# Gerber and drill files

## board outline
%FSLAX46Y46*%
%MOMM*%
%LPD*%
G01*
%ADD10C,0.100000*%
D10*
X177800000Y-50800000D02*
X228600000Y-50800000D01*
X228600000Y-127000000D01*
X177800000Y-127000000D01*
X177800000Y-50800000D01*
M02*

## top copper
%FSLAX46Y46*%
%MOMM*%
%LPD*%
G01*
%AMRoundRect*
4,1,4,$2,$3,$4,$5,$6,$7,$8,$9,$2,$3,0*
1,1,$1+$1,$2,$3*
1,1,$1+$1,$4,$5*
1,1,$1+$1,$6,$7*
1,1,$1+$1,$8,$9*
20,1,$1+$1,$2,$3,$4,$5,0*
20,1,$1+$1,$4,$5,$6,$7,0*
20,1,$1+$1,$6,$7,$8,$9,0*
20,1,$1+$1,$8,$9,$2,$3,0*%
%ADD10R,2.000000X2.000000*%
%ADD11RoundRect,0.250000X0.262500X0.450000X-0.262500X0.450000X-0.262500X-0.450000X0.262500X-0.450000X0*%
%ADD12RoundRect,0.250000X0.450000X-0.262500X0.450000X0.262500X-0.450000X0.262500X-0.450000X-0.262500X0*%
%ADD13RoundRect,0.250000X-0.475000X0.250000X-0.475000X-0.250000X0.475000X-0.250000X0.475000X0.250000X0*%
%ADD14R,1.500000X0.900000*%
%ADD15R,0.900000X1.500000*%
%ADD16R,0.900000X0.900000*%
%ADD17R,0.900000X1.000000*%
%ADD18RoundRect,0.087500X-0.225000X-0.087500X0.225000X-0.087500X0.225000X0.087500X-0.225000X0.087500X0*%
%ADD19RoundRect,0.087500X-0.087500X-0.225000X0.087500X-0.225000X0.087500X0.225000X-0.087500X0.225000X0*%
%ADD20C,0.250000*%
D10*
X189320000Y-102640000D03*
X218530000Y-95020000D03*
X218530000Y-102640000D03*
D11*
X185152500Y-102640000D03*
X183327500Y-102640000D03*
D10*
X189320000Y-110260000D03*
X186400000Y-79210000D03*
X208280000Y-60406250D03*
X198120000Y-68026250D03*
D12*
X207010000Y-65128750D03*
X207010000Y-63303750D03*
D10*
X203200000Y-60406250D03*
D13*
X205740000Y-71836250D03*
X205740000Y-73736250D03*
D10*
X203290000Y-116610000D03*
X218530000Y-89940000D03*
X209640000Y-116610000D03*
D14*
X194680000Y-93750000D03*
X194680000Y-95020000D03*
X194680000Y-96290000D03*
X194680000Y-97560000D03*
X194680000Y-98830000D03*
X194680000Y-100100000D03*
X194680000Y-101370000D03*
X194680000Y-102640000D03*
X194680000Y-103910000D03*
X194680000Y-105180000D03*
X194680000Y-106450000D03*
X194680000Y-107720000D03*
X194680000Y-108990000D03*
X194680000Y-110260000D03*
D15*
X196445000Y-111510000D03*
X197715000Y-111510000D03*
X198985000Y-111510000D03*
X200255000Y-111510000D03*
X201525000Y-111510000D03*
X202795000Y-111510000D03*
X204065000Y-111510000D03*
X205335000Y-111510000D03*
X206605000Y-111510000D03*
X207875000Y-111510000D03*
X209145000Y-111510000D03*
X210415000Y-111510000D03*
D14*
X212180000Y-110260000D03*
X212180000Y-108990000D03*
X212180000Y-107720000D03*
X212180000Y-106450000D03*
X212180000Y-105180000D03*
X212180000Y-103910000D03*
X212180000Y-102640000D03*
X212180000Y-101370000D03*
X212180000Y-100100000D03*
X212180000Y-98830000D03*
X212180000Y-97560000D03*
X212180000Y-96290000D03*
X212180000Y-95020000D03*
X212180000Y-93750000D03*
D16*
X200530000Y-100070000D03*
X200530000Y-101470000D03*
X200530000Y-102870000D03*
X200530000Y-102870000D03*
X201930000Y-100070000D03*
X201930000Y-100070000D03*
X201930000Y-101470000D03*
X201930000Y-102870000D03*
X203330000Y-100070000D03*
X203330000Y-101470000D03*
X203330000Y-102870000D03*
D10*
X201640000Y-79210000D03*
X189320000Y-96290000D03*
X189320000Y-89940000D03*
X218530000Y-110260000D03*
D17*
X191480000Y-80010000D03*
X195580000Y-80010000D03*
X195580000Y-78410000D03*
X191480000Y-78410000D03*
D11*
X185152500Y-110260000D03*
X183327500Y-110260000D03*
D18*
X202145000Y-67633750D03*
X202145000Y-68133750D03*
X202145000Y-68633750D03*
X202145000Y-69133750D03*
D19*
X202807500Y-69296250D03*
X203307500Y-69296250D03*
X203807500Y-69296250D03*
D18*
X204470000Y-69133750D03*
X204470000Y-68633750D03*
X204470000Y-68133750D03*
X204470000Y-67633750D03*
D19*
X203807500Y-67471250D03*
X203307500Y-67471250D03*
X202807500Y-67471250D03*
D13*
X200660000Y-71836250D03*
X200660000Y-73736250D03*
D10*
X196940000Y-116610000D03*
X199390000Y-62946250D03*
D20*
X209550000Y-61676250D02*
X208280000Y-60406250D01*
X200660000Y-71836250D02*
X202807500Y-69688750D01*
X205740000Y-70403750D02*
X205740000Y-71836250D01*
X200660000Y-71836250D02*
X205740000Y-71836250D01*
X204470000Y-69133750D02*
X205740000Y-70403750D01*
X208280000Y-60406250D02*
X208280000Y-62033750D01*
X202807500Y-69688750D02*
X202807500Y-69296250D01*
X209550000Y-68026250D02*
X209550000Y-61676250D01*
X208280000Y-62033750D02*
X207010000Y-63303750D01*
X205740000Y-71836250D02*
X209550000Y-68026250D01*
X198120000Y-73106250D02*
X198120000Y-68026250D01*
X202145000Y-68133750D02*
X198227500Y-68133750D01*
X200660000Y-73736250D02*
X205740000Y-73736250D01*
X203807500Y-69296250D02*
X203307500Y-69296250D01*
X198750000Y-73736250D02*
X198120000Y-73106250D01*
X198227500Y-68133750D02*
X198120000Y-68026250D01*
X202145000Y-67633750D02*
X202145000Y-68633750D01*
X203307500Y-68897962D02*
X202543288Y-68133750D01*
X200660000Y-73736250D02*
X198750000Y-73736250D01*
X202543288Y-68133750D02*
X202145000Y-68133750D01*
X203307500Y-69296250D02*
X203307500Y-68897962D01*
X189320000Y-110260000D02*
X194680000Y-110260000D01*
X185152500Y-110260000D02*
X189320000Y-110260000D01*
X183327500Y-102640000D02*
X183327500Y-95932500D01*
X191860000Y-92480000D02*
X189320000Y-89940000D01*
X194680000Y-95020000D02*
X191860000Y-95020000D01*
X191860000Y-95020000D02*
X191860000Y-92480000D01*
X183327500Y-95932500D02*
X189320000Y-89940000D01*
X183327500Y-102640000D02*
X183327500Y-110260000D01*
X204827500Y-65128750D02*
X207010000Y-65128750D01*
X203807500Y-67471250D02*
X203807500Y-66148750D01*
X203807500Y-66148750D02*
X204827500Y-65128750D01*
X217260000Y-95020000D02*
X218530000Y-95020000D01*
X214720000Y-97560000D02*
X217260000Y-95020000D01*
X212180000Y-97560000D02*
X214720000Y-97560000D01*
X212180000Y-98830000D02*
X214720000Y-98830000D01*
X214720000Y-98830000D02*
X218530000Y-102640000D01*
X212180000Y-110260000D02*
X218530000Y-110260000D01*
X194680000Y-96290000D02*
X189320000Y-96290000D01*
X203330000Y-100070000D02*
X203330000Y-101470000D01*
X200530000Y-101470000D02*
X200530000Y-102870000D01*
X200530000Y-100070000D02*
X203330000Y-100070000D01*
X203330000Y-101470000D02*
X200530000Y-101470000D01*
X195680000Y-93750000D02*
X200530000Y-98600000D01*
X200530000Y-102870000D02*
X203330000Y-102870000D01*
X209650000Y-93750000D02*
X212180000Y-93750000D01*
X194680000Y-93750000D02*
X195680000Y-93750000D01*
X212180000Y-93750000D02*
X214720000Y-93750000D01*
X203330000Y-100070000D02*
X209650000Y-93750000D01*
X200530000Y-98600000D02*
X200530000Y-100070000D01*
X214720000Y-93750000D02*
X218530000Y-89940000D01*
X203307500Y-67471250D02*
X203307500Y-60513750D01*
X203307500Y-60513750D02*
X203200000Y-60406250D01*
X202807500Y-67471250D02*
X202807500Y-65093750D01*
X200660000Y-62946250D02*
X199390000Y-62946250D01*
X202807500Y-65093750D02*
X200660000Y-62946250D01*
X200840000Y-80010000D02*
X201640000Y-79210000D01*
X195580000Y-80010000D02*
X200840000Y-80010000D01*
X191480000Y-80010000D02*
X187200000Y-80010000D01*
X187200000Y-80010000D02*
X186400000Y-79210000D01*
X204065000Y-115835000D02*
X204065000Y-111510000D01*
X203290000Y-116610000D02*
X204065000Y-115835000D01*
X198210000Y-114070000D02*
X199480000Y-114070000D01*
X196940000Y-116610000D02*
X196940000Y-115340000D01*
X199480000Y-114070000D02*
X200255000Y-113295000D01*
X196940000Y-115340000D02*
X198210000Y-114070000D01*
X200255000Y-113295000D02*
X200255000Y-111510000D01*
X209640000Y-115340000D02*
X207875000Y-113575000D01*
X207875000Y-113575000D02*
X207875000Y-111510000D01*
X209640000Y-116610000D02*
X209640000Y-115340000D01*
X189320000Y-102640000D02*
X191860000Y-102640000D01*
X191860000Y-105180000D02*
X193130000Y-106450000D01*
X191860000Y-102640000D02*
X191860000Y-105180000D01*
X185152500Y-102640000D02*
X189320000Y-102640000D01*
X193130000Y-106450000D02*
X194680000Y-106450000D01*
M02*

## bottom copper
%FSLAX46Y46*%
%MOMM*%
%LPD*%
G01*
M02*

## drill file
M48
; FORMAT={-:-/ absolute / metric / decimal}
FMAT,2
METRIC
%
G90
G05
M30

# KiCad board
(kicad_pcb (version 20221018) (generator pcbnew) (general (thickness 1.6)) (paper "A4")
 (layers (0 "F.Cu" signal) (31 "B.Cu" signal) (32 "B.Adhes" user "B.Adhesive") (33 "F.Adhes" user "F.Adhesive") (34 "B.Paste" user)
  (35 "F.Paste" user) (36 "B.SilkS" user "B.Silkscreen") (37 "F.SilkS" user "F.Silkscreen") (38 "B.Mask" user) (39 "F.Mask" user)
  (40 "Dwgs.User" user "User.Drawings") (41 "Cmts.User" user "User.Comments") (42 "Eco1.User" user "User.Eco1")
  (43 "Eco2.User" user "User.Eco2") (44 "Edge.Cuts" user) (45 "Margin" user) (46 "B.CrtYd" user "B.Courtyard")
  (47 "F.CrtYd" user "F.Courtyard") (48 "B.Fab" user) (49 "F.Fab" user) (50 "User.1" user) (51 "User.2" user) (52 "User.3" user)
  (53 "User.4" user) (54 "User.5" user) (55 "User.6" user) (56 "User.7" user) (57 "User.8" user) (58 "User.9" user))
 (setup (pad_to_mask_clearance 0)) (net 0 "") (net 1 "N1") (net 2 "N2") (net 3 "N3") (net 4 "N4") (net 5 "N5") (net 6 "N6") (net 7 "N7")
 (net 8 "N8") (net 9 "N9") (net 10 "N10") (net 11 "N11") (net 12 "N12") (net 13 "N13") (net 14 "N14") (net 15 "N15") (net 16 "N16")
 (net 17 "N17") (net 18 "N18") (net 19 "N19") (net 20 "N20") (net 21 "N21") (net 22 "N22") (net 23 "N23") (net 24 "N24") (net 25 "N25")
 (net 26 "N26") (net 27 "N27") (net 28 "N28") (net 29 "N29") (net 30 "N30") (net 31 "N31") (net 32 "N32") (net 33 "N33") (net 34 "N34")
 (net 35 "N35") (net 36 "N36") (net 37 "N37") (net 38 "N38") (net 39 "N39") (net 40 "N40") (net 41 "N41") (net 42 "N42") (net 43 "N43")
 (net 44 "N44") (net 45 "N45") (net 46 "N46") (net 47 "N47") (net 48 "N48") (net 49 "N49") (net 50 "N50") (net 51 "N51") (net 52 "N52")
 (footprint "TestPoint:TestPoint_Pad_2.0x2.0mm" (layer "F.Cu") (at 189.32 102.64)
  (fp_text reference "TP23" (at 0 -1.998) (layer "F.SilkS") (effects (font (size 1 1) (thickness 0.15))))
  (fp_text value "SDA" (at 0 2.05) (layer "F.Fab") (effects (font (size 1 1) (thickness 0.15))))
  (pad "1" smd rect (at 0 0) (size 2 2) (layers "F.Cu" "F.Mask") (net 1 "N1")))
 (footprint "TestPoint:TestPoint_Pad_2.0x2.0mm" (layer "F.Cu") (at 218.53 95.02)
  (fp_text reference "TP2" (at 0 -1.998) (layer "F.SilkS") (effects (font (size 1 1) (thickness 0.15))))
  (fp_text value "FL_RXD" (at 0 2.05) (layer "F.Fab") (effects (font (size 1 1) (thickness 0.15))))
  (pad "1" smd rect (at 0 0) (size 2 2) (layers "F.Cu" "F.Mask") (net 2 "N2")))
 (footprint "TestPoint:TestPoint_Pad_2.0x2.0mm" (layer "F.Cu") (at 218.53 102.64)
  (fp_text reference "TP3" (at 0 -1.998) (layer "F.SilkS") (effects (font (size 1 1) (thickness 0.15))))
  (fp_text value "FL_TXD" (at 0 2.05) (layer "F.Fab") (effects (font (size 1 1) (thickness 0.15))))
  (pad "1" smd rect (at 0 0) (size 2 2) (layers "F.Cu" "F.Mask") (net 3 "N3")))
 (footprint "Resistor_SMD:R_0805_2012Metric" (layer "F.Cu") (at 184.24 102.64 180)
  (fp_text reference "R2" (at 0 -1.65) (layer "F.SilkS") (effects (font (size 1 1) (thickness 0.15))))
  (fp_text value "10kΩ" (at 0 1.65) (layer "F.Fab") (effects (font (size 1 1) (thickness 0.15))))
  (pad "1" smd roundrect (at -0.9125 0 180) (size 1.025 1.4) (layers "F.Cu" "F.Paste" "F.Mask") (roundrect_rratio 0.243902) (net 1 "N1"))
  (pad "2" smd roundrect (at 0.9125 0 180) (size 1.025 1.4) (layers "F.Cu" "F.Paste" "F.Mask") (roundrect_rratio 0.243902) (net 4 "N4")))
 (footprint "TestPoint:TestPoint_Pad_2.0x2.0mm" (layer "F.Cu") (at 189.32 110.26)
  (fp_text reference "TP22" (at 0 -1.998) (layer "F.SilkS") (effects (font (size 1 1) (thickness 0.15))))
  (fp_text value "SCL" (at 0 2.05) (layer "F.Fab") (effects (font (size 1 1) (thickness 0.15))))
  (pad "1" smd rect (at 0 0) (size 2 2) (layers "F.Cu" "F.Mask") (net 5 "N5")))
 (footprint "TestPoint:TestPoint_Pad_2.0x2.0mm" (layer "F.Cu") (at 186.4 79.21)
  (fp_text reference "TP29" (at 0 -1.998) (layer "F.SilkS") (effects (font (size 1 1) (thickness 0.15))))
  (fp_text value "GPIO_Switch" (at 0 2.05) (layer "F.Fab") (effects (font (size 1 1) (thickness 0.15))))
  (pad "1" smd rect (at 0 0) (size 2 2) (layers "F.Cu" "F.Mask") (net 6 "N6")))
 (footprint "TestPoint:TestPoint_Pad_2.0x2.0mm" (layer "F.Cu") (at 208.28 60.40625)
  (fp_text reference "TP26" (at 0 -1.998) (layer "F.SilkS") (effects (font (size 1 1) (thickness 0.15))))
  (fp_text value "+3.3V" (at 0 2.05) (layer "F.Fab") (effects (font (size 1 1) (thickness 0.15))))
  (pad "1" smd rect (at 0 0) (size 2 2) (layers "F.Cu" "F.Mask") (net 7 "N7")))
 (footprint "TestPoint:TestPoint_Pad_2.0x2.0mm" (layer "F.Cu") (at 198.12 68.02625)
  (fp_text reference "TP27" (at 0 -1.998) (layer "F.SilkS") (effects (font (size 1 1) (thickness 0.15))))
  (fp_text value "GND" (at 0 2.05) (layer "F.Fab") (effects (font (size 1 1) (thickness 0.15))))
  (pad "1" smd rect (at 0 0) (size 2 2) (layers "F.Cu" "F.Mask") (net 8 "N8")))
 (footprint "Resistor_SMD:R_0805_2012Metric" (layer "F.Cu") (at 207.01 64.21625 90)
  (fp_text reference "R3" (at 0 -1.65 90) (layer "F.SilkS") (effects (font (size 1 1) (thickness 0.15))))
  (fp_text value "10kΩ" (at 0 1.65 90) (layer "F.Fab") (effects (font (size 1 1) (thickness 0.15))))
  (pad "1" smd roundrect (at -0.9125 0 90) (size 1.025 1.4) (layers "F.Cu" "F.Paste" "F.Mask") (roundrect_rratio 0.243902) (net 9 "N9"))
  (pad "2" smd roundrect (at 0.9125 0 90) (size 1.025 1.4) (layers "F.Cu" "F.Paste" "F.Mask") (roundrect_rratio 0.243902) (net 7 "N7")))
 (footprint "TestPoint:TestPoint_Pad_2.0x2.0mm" (layer "F.Cu") (at 203.2 60.40625)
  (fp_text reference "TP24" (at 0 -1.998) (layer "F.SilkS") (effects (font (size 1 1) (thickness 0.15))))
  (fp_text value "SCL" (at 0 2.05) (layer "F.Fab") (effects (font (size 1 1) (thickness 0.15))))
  (pad "1" smd rect (at 0 0) (size 2 2) (layers "F.Cu" "F.Mask") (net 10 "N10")))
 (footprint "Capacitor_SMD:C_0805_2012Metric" (layer "F.Cu") (at 205.74 72.78625 -90)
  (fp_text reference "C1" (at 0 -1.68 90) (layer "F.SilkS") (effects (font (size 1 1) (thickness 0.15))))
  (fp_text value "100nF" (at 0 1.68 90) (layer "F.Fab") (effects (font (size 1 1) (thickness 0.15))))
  (pad "1" smd roundrect (at -0.95 0 270) (size 1 1.45) (layers "F.Cu" "F.Paste" "F.Mask") (roundrect_rratio 0.25) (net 7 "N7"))
  (pad "2" smd roundrect (at 0.95 0 270) (size 1 1.45) (layers "F.Cu" "F.Paste" "F.Mask") (roundrect_rratio 0.25) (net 8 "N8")))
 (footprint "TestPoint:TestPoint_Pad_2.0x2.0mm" (layer "F.Cu") (at 203.29 116.61)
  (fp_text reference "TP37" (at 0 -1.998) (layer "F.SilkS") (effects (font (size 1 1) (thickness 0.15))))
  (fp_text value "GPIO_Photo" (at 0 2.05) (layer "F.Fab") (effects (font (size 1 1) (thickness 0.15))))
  (pad "1" smd rect (at 0 0) (size 2 2) (layers "F.Cu" "F.Mask") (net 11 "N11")))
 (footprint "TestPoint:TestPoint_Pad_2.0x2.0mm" (layer "F.Cu") (at 218.53 89.94)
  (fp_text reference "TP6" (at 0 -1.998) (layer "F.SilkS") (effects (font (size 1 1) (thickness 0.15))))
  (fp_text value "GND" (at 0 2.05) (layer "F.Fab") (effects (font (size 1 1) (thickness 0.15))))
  (pad "1" smd rect (at 0 0) (size 2 2) (layers "F.Cu" "F.Mask") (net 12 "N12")))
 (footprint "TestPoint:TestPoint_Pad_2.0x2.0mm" (layer "F.Cu") (at 209.64 116.61)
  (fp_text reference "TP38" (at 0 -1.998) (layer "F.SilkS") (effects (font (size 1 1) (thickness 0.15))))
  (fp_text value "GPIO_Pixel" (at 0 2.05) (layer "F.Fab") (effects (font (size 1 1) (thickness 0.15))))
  (pad "1" smd rect (at 0 0) (size 2 2) (layers "F.Cu" "F.Mask") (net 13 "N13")))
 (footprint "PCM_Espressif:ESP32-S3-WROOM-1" (layer "F.Cu") (at 203.43 102.01)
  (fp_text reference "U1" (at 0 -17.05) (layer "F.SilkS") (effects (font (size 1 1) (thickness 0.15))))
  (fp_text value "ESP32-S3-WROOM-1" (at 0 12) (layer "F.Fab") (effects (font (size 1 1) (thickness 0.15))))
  (pad "1" smd rect (at -8.75 -8.26) (size 1.5 0.9) (layers "F.Cu" "F.Paste" "F.Mask") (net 12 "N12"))
  (pad "2" smd rect (at -8.75 -6.99) (size 1.5 0.9) (layers "F.Cu" "F.Paste" "F.Mask") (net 4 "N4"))
  (pad "3" smd rect (at -8.75 -5.72) (size 1.5 0.9) (layers "F.Cu" "F.Paste" "F.Mask") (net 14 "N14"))
  (pad "4" smd rect (at -8.75 -4.45) (size 1.5 0.9) (layers "F.Cu" "F.Paste" "F.Mask") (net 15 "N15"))
  (pad "5" smd rect (at -8.75 -3.18) (size 1.5 0.9) (layers "F.Cu" "F.Paste" "F.Mask") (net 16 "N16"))
  (pad "6" smd rect (at -8.75 -1.91) (size 1.5 0.9) (layers "F.Cu" "F.Paste" "F.Mask") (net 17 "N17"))
  (pad "7" smd rect (at -8.75 -0.64) (size 1.5 0.9) (layers "F.Cu" "F.Paste" "F.Mask") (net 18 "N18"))
  (pad "8" smd rect (at -8.75 0.63) (size 1.5 0.9) (layers "F.Cu" "F.Paste" "F.Mask") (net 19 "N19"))
  (pad "9" smd rect (at -8.75 1.9) (size 1.5 0.9) (layers "F.Cu" "F.Paste" "F.Mask") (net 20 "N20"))
  (pad "10" smd rect (at -8.75 3.17) (size 1.5 0.9) (layers "F.Cu" "F.Paste" "F.Mask") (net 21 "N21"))
  (pad "11" smd rect (at -8.75 4.44) (size 1.5 0.9) (layers "F.Cu" "F.Paste" "F.Mask") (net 1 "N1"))
  (pad "12" smd rect (at -8.75 5.71) (size 1.5 0.9) (layers "F.Cu" "F.Paste" "F.Mask") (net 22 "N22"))
  (pad "13" smd rect (at -8.75 6.98) (size 1.5 0.9) (layers "F.Cu" "F.Paste" "F.Mask") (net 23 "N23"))
  (pad "14" smd rect (at -8.75 8.25) (size 1.5 0.9) (layers "F.Cu" "F.Paste" "F.Mask") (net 5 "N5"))
  (pad "15" smd rect (at -6.985 9.5 90) (size 1.5 0.9) (layers "F.Cu" "F.Paste" "F.Mask") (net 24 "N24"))
  (pad "16" smd rect (at -5.715 9.5 90) (size 1.5 0.9) (layers "F.Cu" "F.Paste" "F.Mask") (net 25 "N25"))
  (pad "17" smd rect (at -4.445 9.5 90) (size 1.5 0.9) (layers "F.Cu" "F.Paste" "F.Mask") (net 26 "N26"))
  (pad "18" smd rect (at -3.175 9.5 90) (size 1.5 0.9) (layers "F.Cu" "F.Paste" "F.Mask") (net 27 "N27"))
  (pad "19" smd rect (at -1.905 9.5 90) (size 1.5 0.9) (layers "F.Cu" "F.Paste" "F.Mask") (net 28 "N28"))
  (pad "20" smd rect (at -0.635 9.5 90) (size 1.5 0.9) (layers "F.Cu" "F.Paste" "F.Mask") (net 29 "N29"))
  (pad "21" smd rect (at 0.635 9.5 90) (size 1.5 0.9) (layers "F.Cu" "F.Paste" "F.Mask") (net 11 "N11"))
  (pad "22" smd rect (at 1.905 9.5 90) (size 1.5 0.9) (layers "F.Cu" "F.Paste" "F.Mask") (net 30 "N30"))
  (pad "23" smd rect (at 3.175 9.5 90) (size 1.5 0.9) (layers "F.Cu" "F.Paste" "F.Mask") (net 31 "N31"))
  (pad "24" smd rect (at 4.445 9.5 90) (size 1.5 0.9) (layers "F.Cu" "F.Paste" "F.Mask") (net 13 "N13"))
  (pad "25" smd rect (at 5.715 9.5 90) (size 1.5 0.9) (layers "F.Cu" "F.Paste" "F.Mask") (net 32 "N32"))
  (pad "26" smd rect (at 6.985 9.5 90) (size 1.5 0.9) (layers "F.Cu" "F.Paste" "F.Mask") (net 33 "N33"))
  (pad "27" smd rect (at 8.75 8.25 180) (size 1.5 0.9) (layers "F.Cu" "F.Paste" "F.Mask") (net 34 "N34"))
  (pad "28" smd rect (at 8.75 6.98 180) (size 1.5 0.9) (layers "F.Cu" "F.Paste" "F.Mask") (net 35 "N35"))
  (pad "29" smd rect (at 8.75 5.71 180) (size 1.5 0.9) (layers "F.Cu" "F.Paste" "F.Mask") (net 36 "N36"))
  (pad "30" smd rect (at 8.75 4.44 180) (size 1.5 0.9) (layers "F.Cu" "F.Paste" "F.Mask") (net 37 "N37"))
  (pad "31" smd rect (at 8.75 3.17 180) (size 1.5 0.9) (layers "F.Cu" "F.Paste" "F.Mask") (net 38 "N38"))
  (pad "32" smd rect (at 8.75 1.9 180) (size 1.5 0.9) (layers "F.Cu" "F.Paste" "F.Mask") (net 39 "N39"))
  (pad "33" smd rect (at 8.75 0.63 180) (size 1.5 0.9) (layers "F.Cu" "F.Paste" "F.Mask") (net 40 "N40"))
  (pad "34" smd rect (at 8.75 -0.64 180) (size 1.5 0.9) (layers "F.Cu" "F.Paste" "F.Mask") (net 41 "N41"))
  (pad "35" smd rect (at 8.75 -1.91 180) (size 1.5 0.9) (layers "F.Cu" "F.Paste" "F.Mask") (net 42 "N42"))
  (pad "36" smd rect (at 8.75 -3.18 180) (size 1.5 0.9) (layers "F.Cu" "F.Paste" "F.Mask") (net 3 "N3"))
  (pad "37" smd rect (at 8.75 -4.45 180) (size 1.5 0.9) (layers "F.Cu" "F.Paste" "F.Mask") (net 2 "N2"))
  (pad "38" smd rect (at 8.75 -5.72 180) (size 1.5 0.9) (layers "F.Cu" "F.Paste" "F.Mask") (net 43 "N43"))
  (pad "39" smd rect (at 8.75 -6.99 180) (size 1.5 0.9) (layers "F.Cu" "F.Paste" "F.Mask") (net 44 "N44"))
  (pad "40" smd rect (at 8.75 -8.26 180) (size 1.5 0.9) (layers "F.Cu" "F.Paste" "F.Mask") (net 12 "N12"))
  (pad "41" smd rect (at -2.9 -1.94 180) (size 0.9 0.9) (layers "F.Cu" "F.Paste" "F.Mask") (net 12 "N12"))
  (pad "41" smd rect (at -2.9 -0.54 180) (size 0.9 0.9) (layers "F.Cu" "F.Paste" "F.Mask") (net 12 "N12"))
  (pad "41" smd rect (at -2.9 0.86 180) (size 0.9 0.9) (layers "F.Cu" "F.Paste" "F.Mask") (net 12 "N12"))
  (pad "41" smd rect (at -2.9 0.86 180) (size 0.9 0.9) (layers "F.Cu" "F.Paste" "F.Mask") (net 12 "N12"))
  (pad "41" smd rect (at -1.5 -1.94 180) (size 0.9 0.9) (layers "F.Cu" "F.Paste" "F.Mask") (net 12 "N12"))
  (pad "41" smd rect (at -1.5 -1.94 180) (size 0.9 0.9) (layers "F.Cu" "F.Paste" "F.Mask") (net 12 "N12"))
  (pad "41" smd rect (at -1.5 -0.54 180) (size 0.9 0.9) (layers "F.Cu" "F.Paste" "F.Mask") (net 12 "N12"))
  (pad "41" smd rect (at -1.5 0.86 180) (size 0.9 0.9) (layers "F.Cu" "F.Paste" "F.Mask") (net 12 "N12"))
  (pad "41" smd rect (at -0.1 -1.94 180) (size 0.9 0.9) (layers "F.Cu" "F.Paste" "F.Mask") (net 12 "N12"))
  (pad "41" smd rect (at -0.1 -0.54 180) (size 0.9 0.9) (layers "F.Cu" "F.Paste" "F.Mask") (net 12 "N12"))
  (pad "41" smd rect (at -0.1 0.86 180) (size 0.9 0.9) (layers "F.Cu" "F.Paste" "F.Mask") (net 12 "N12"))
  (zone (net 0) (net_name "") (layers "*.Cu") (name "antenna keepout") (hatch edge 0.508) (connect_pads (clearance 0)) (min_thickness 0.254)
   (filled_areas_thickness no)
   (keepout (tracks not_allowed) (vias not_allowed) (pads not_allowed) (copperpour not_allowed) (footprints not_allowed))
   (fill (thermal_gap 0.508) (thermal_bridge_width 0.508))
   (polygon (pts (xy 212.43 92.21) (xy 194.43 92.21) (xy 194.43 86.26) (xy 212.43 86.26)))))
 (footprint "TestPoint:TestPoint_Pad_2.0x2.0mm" (layer "F.Cu") (at 201.64 79.21)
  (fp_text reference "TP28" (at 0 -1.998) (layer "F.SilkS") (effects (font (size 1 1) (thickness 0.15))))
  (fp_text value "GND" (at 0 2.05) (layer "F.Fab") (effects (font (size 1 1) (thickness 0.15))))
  (pad "1" smd rect (at 0 0) (size 2 2) (layers "F.Cu" "F.Mask") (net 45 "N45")))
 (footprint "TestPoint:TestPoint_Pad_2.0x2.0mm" (layer "F.Cu") (at 189.32 96.29)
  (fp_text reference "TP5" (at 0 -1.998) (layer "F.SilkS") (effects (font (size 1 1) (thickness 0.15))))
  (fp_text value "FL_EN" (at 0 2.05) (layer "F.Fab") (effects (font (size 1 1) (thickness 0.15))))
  (pad "1" smd rect (at 0 0) (size 2 2) (layers "F.Cu" "F.Mask") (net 14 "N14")))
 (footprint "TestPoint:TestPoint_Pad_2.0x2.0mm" (layer "F.Cu") (at 189.32 89.94)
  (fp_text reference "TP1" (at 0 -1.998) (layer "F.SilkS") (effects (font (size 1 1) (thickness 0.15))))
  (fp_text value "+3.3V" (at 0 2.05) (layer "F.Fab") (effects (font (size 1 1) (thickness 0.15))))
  (pad "1" smd rect (at 0 0) (size 2 2) (layers "F.Cu" "F.Mask") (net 4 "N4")))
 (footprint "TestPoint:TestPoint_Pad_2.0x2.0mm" (layer "F.Cu") (at 218.53 110.26)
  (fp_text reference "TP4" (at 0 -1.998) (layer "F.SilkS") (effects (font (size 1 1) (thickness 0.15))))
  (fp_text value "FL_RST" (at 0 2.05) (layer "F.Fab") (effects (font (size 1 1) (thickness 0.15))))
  (pad "1" smd rect (at 0 0) (size 2 2) (layers "F.Cu" "F.Mask") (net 34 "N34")))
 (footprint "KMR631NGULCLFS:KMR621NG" (layer "F.Cu") (at 193.53 79.21)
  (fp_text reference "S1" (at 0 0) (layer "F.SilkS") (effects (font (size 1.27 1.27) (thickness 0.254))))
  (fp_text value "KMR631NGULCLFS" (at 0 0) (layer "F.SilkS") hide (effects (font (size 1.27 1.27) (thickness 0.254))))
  (pad "1" smd rect (at -2.05 0.8) (size 0.9 1) (layers "F.Cu" "F.Paste" "F.Mask") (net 6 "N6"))
  (pad "2" smd rect (at 2.05 0.8) (size 0.9 1) (layers "F.Cu" "F.Paste" "F.Mask") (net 45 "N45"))
  (pad "3" smd rect (at 2.05 -0.8) (size 0.9 1) (layers "F.Cu" "F.Paste" "F.Mask") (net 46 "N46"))
  (pad "4" smd rect (at -2.05 -0.8) (size 0.9 1) (layers "F.Cu" "F.Paste" "F.Mask") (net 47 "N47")))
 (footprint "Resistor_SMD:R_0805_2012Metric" (layer "F.Cu") (at 184.24 110.26 180)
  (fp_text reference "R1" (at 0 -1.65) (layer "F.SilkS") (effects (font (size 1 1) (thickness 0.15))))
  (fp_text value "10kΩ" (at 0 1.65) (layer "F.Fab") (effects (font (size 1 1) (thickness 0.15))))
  (pad "1" smd roundrect (at -0.9125 0 180) (size 1.025 1.4) (layers "F.Cu" "F.Paste" "F.Mask") (roundrect_rratio 0.243902) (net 5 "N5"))
  (pad "2" smd roundrect (at 0.9125 0 180) (size 1.025 1.4) (layers "F.Cu" "F.Paste" "F.Mask") (roundrect_rratio 0.243902) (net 4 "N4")))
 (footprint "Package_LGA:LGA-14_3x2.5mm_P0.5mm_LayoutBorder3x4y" (layer "F.Cu") (at 203.3075 68.38375)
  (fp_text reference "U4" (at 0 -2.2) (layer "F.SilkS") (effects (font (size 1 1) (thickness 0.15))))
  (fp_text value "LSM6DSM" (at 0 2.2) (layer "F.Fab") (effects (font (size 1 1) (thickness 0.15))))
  (pad "1" smd roundrect (at -1.1625 -0.75) (size 0.625 0.35) (layers "F.Cu" "F.Paste" "F.Mask") (roundrect_rratio 0.25) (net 8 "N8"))
  (pad "2" smd roundrect (at -1.1625 -0.25) (size 0.625 0.35) (layers "F.Cu" "F.Paste" "F.Mask") (roundrect_rratio 0.25) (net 8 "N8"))
  (pad "3" smd roundrect (at -1.1625 0.25) (size 0.625 0.35) (layers "F.Cu" "F.Paste" "F.Mask") (roundrect_rratio 0.25) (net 8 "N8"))
  (pad "4" smd roundrect (at -1.1625 0.75) (size 0.625 0.35) (layers "F.Cu" "F.Paste" "F.Mask") (roundrect_rratio 0.25) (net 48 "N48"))
  (pad "5" smd roundrect (at -0.5 0.9125) (size 0.35 0.625) (layers "F.Cu" "F.Paste" "F.Mask") (roundrect_rratio 0.25) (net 7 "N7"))
  (pad "6" smd roundrect (at 0 0.9125) (size 0.35 0.625) (layers "F.Cu" "F.Paste" "F.Mask") (roundrect_rratio 0.25) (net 8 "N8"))
  (pad "7" smd roundrect (at 0.5 0.9125) (size 0.35 0.625) (layers "F.Cu" "F.Paste" "F.Mask") (roundrect_rratio 0.25) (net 8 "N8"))
  (pad "8" smd roundrect (at 1.1625 0.75) (size 0.625 0.35) (layers "F.Cu" "F.Paste" "F.Mask") (roundrect_rratio 0.25) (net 7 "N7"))
  (pad "9" smd roundrect (at 1.1625 0.25) (size 0.625 0.35) (layers "F.Cu" "F.Paste" "F.Mask") (roundrect_rratio 0.25) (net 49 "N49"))
  (pad "10" smd roundrect (at 1.1625 -0.25) (size 0.625 0.35) (layers "F.Cu" "F.Paste" "F.Mask") (roundrect_rratio 0.25) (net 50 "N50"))
  (pad "11" smd roundrect (at 1.1625 -0.75) (size 0.625 0.35) (layers "F.Cu" "F.Paste" "F.Mask") (roundrect_rratio 0.25) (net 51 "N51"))
  (pad "12" smd roundrect (at 0.5 -0.9125) (size 0.35 0.625) (layers "F.Cu" "F.Paste" "F.Mask") (roundrect_rratio 0.25) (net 9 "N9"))
  (pad "13" smd roundrect (at 0 -0.9125) (size 0.35 0.625) (layers "F.Cu" "F.Paste" "F.Mask") (roundrect_rratio 0.25) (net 10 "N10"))
  (pad "14" smd roundrect (at -0.5 -0.9125) (size 0.35 0.625) (layers "F.Cu" "F.Paste" "F.Mask") (roundrect_rratio 0.25) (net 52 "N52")))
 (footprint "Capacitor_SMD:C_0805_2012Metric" (layer "F.Cu") (at 200.66 72.78625 -90)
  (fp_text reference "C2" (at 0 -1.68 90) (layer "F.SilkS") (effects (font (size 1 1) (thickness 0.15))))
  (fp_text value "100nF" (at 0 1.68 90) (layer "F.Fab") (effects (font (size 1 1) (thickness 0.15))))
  (pad "1" smd roundrect (at -0.95 0 270) (size 1 1.45) (layers "F.Cu" "F.Paste" "F.Mask") (roundrect_rratio 0.25) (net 7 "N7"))
  (pad "2" smd roundrect (at 0.95 0 270) (size 1 1.45) (layers "F.Cu" "F.Paste" "F.Mask") (roundrect_rratio 0.25) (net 8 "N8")))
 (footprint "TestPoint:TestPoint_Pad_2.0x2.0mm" (layer "F.Cu") (at 196.94 116.61)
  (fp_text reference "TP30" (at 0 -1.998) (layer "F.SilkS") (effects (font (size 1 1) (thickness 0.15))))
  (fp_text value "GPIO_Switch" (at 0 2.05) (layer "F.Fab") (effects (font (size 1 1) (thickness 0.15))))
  (pad "1" smd rect (at 0 0) (size 2 2) (layers "F.Cu" "F.Mask") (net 27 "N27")))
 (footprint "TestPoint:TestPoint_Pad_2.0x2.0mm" (layer "F.Cu") (at 199.39 62.94625)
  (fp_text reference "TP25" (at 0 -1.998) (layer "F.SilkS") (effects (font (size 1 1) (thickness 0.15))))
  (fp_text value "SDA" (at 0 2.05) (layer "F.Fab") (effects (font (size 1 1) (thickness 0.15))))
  (pad "1" smd rect (at 0 0) (size 2 2) (layers "F.Cu" "F.Mask") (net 52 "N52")))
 (gr_rect (start 177.8 50.8) (end 228.6 127) (stroke (width 0.1) (type default)) (fill none) (layer "Edge.Cuts"))
 (segment (start 209.55 61.67625) (end 208.28 60.40625) (width 0.25) (layer "F.Cu") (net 7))
 (segment (start 200.66 71.83625) (end 202.8075 69.68875) (width 0.25) (layer "F.Cu") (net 7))
 (segment (start 205.74 70.40375) (end 205.74 71.83625) (width 0.25) (layer "F.Cu") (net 7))
 (segment (start 200.66 71.83625) (end 205.74 71.83625) (width 0.25) (layer "F.Cu") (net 7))
 (segment (start 204.47 69.13375) (end 205.74 70.40375) (width 0.25) (layer "F.Cu") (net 7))
 (segment (start 208.28 60.40625) (end 208.28 62.03375) (width 0.25) (layer "F.Cu") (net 7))
 (segment (start 202.8075 69.68875) (end 202.8075 69.29625) (width 0.25) (layer "F.Cu") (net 7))
 (segment (start 209.55 68.02625) (end 209.55 61.67625) (width 0.25) (layer "F.Cu") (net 7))
 (segment (start 208.28 62.03375) (end 207.01 63.30375) (width 0.25) (layer "F.Cu") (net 7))
 (segment (start 205.74 71.83625) (end 209.55 68.02625) (width 0.25) (layer "F.Cu") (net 7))
 (segment (start 198.12 73.10625) (end 198.12 68.02625) (width 0.25) (layer "F.Cu") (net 8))
 (segment (start 202.145 68.13375) (end 198.2275 68.13375) (width 0.25) (layer "F.Cu") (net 8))
 (segment (start 200.66 73.73625) (end 205.74 73.73625) (width 0.25) (layer "F.Cu") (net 8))
 (segment (start 203.8075 69.29625) (end 203.3075 69.29625) (width 0.25) (layer "F.Cu") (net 8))
 (segment (start 198.75 73.73625) (end 198.12 73.10625) (width 0.25) (layer "F.Cu") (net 8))
 (segment (start 198.2275 68.13375) (end 198.12 68.02625) (width 0.25) (layer "F.Cu") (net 8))
 (segment (start 202.145 67.63375) (end 202.145 68.63375) (width 0.25) (layer "F.Cu") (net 8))
 (segment (start 203.3075 68.897962) (end 202.543288 68.13375) (width 0.25) (layer "F.Cu") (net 8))
 (segment (start 200.66 73.73625) (end 198.75 73.73625) (width 0.25) (layer "F.Cu") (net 8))
 (segment (start 202.543288 68.13375) (end 202.145 68.13375) (width 0.25) (layer "F.Cu") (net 8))
 (segment (start 203.3075 69.29625) (end 203.3075 68.897962) (width 0.25) (layer "F.Cu") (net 8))
 (segment (start 189.32 110.26) (end 194.68 110.26) (width 0.25) (layer "F.Cu") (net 5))
 (segment (start 185.1525 110.26) (end 189.32 110.26) (width 0.25) (layer "F.Cu") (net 5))
 (segment (start 183.3275 102.64) (end 183.3275 95.9325) (width 0.25) (layer "F.Cu") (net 4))
 (segment (start 191.86 92.48) (end 189.32 89.94) (width 0.25) (layer "F.Cu") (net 4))
 (segment (start 194.68 95.02) (end 191.86 95.02) (width 0.25) (layer "F.Cu") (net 4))
 (segment (start 191.86 95.02) (end 191.86 92.48) (width 0.25) (layer "F.Cu") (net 4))
 (segment (start 183.3275 95.9325) (end 189.32 89.94) (width 0.25) (layer "F.Cu") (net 4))
 (segment (start 183.3275 102.64) (end 183.3275 110.26) (width 0.25) (layer "F.Cu") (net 4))
 (segment (start 204.8275 65.12875) (end 207.01 65.12875) (width 0.25) (layer "F.Cu") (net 9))
 (segment (start 203.8075 67.47125) (end 203.8075 66.14875) (width 0.25) (layer "F.Cu") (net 9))
 (segment (start 203.8075 66.14875) (end 204.8275 65.12875) (width 0.25) (layer "F.Cu") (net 9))
 (segment (start 217.26 95.02) (end 218.53 95.02) (width 0.25) (layer "F.Cu") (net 2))
 (segment (start 214.72 97.56) (end 217.26 95.02) (width 0.25) (layer "F.Cu") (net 2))
 (segment (start 212.18 97.56) (end 214.72 97.56) (width 0.25) (layer "F.Cu") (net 2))
 (segment (start 212.18 98.83) (end 214.72 98.83) (width 0.25) (layer "F.Cu") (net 3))
 (segment (start 214.72 98.83) (end 218.53 102.64) (width 0.25) (layer "F.Cu") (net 3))
 (segment (start 212.18 110.26) (end 218.53 110.26) (width 0.25) (layer "F.Cu") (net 34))
 (segment (start 194.68 96.29) (end 189.32 96.29) (width 0.25) (layer "F.Cu") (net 14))
 (segment (start 203.33 100.07) (end 203.33 101.47) (width 0.25) (layer "F.Cu") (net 12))
 (segment (start 200.53 101.47) (end 200.53 102.87) (width 0.25) (layer "F.Cu") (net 12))
 (segment (start 200.53 100.07) (end 203.33 100.07) (width 0.25) (layer "F.Cu") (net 12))
 (segment (start 203.33 101.47) (end 200.53 101.47) (width 0.25) (layer "F.Cu") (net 12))
 (segment (start 195.68 93.75) (end 200.53 98.6) (width 0.25) (layer "F.Cu") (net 12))
 (segment (start 200.53 102.87) (end 203.33 102.87) (width 0.25) (layer "F.Cu") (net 12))
 (segment (start 209.65 93.75) (end 212.18 93.75) (width 0.25) (layer "F.Cu") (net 12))
 (segment (start 194.68 93.75) (end 195.68 93.75) (width 0.25) (layer "F.Cu") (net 12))
 (segment (start 212.18 93.75) (end 214.72 93.75) (width 0.25) (layer "F.Cu") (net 12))
 (segment (start 203.33 100.07) (end 209.65 93.75) (width 0.25) (layer "F.Cu") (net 12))
 (segment (start 200.53 98.6) (end 200.53 100.07) (width 0.25) (layer "F.Cu") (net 12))
 (segment (start 214.72 93.75) (end 218.53 89.94) (width 0.25) (layer "F.Cu") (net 12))
 (segment (start 203.3075 67.47125) (end 203.3075 60.51375) (width 0.25) (layer "F.Cu") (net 10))
 (segment (start 203.3075 60.51375) (end 203.2 60.40625) (width 0.25) (layer "F.Cu") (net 10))
 (segment (start 202.8075 67.47125) (end 202.8075 65.09375) (width 0.25) (layer "F.Cu") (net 52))
 (segment (start 200.66 62.94625) (end 199.39 62.94625) (width 0.25) (layer "F.Cu") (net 52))
 (segment (start 202.8075 65.09375) (end 200.66 62.94625) (width 0.25) (layer "F.Cu") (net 52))
 (segment (start 200.84 80.01) (end 201.64 79.21) (width 0.25) (layer "F.Cu") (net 45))
 (segment (start 195.58 80.01) (end 200.84 80.01) (width 0.25) (layer "F.Cu") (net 45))
 (segment (start 191.48 80.01) (end 187.2 80.01) (width 0.25) (layer "F.Cu") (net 6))
 (segment (start 187.2 80.01) (end 186.4 79.21) (width 0.25) (layer "F.Cu") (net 6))
 (segment (start 204.065 115.835) (end 204.065 111.51) (width 0.25) (layer "F.Cu") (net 11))
 (segment (start 203.29 116.61) (end 204.065 115.835) (width 0.25) (layer "F.Cu") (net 11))
 (segment (start 198.21 114.07) (end 199.48 114.07) (width 0.25) (layer "F.Cu") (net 27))
 (segment (start 196.94 116.61) (end 196.94 115.34) (width 0.25) (layer "F.Cu") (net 27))
 (segment (start 199.48 114.07) (end 200.255 113.295) (width 0.25) (layer "F.Cu") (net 27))
 (segment (start 196.94 115.34) (end 198.21 114.07) (width 0.25) (layer "F.Cu") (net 27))
 (segment (start 200.255 113.295) (end 200.255 111.51) (width 0.25) (layer "F.Cu") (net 27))
 (segment (start 209.64 115.34) (end 207.875 113.575) (width 0.25) (layer "F.Cu") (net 13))
 (segment (start 207.875 113.575) (end 207.875 111.51) (width 0.25) (layer "F.Cu") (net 13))
 (segment (start 209.64 116.61) (end 209.64 115.34) (width 0.25) (layer "F.Cu") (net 13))
 (segment (start 189.32 102.64) (end 191.86 102.64) (width 0.25) (layer "F.Cu") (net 1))
 (segment (start 191.86 105.18) (end 193.13 106.45) (width 0.25) (layer "F.Cu") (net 1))
 (segment (start 191.86 102.64) (end 191.86 105.18) (width 0.25) (layer "F.Cu") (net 1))
 (segment (start 185.1525 102.64) (end 189.32 102.64) (width 0.25) (layer "F.Cu") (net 1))
 (segment (start 193.13 106.45) (end 194.68 106.45) (width 0.25) (layer "F.Cu") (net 1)))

